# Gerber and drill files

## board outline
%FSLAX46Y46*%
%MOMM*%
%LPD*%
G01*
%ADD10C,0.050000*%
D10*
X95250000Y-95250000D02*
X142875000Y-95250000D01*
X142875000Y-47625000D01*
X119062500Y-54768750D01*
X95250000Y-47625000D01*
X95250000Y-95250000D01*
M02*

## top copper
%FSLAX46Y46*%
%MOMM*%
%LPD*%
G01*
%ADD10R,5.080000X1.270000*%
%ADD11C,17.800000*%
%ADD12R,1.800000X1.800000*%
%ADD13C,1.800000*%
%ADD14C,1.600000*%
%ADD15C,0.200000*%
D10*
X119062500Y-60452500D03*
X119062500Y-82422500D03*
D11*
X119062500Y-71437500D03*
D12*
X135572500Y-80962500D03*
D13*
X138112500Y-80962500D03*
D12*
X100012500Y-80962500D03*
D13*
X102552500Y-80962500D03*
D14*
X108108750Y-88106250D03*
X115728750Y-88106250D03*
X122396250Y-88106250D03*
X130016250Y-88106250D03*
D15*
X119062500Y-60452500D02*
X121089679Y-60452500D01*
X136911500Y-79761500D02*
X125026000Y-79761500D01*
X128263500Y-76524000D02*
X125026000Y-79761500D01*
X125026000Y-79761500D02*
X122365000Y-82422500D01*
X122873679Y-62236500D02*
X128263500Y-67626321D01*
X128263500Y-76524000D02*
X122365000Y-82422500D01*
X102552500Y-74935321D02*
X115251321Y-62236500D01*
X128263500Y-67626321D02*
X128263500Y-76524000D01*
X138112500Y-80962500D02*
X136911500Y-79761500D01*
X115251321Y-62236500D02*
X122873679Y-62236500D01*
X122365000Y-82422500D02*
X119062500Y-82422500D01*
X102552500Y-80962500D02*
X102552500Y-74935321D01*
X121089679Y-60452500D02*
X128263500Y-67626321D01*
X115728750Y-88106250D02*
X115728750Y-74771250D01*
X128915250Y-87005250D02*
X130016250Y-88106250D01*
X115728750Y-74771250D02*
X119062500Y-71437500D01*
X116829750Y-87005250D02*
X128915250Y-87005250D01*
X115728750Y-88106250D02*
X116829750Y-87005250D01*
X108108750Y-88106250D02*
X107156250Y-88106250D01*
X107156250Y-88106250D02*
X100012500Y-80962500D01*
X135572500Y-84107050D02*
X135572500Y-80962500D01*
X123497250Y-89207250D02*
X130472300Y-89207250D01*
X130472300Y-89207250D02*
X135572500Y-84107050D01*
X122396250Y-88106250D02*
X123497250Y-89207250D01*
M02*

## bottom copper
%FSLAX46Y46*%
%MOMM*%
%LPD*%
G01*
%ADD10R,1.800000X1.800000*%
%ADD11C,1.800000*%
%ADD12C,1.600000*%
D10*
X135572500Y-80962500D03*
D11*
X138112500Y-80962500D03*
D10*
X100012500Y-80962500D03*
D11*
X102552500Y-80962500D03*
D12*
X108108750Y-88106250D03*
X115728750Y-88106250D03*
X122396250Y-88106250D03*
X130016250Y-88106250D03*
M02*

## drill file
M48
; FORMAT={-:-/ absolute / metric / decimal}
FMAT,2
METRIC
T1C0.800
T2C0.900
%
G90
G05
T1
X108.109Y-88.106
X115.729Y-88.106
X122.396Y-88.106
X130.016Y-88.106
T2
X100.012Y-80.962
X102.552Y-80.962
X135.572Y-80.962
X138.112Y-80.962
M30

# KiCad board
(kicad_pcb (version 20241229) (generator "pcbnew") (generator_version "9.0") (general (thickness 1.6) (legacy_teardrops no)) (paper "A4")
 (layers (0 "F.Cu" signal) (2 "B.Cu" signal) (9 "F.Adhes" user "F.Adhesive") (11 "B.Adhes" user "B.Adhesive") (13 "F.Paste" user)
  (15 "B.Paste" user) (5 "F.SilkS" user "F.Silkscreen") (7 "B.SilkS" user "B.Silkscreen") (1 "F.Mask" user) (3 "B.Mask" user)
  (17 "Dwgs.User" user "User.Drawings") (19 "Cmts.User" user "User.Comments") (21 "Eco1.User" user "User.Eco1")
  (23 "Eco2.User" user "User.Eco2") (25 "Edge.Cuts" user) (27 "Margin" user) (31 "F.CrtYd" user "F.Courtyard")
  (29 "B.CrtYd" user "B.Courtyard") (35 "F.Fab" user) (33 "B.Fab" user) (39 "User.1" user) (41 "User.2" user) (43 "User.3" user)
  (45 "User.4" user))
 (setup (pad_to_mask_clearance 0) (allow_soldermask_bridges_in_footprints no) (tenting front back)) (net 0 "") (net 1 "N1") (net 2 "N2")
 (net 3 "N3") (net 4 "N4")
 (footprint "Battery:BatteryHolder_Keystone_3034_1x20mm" (layer "F.Cu") (at 119.0625 71.4375 -90)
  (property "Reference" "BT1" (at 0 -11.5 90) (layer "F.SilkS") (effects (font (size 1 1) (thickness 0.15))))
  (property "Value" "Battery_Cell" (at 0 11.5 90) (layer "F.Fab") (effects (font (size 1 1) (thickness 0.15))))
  (pad "1" smd rect (at -10.985 0 270) (size 1.27 5.08) (layers "F.Cu" "F.Mask" "F.Paste") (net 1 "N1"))
  (pad "1" smd rect (at 10.985 0 270) (size 1.27 5.08) (layers "F.Cu" "F.Mask" "F.Paste") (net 1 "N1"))
  (pad "2" smd circle (at 0 0 270) (size 17.8 17.8) (layers "F.Cu" "F.Mask") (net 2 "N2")))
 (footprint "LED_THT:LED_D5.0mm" (layer "F.Cu") (at 135.5725 80.9625)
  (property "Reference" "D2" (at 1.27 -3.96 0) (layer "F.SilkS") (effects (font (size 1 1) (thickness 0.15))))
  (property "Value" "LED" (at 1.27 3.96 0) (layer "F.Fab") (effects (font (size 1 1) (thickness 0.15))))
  (pad "1" thru_hole rect (at 0 0) (size 1.8 1.8) (drill 0.9) (layers "*.Cu" "*.Mask") (remove_unused_layers no) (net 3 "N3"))
  (pad "2" thru_hole circle (at 2.54 0) (size 1.8 1.8) (drill 0.9) (layers "*.Cu" "*.Mask") (remove_unused_layers no) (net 1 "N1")))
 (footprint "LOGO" (layer "F.Cu") (at 104.775 57.15)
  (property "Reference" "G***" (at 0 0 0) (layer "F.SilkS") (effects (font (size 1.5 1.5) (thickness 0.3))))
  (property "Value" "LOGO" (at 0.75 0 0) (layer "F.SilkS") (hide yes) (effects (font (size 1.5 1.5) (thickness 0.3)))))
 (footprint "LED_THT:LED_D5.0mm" (layer "F.Cu") (at 100.0125 80.9625)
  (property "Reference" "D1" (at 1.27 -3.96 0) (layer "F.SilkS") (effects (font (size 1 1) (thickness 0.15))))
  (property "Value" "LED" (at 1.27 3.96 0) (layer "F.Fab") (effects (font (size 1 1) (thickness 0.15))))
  (pad "1" thru_hole rect (at 0 0) (size 1.8 1.8) (drill 0.9) (layers "*.Cu" "*.Mask") (remove_unused_layers no) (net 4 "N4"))
  (pad "2" thru_hole circle (at 2.54 0) (size 1.8 1.8) (drill 0.9) (layers "*.Cu" "*.Mask") (remove_unused_layers no) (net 1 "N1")))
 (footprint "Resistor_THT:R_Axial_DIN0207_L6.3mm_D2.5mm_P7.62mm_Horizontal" (layer "F.Cu") (at 108.10875 88.10625)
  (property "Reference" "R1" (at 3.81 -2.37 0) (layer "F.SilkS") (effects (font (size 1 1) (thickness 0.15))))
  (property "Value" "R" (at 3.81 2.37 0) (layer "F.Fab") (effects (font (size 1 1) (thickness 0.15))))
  (pad "1" thru_hole circle (at 0 0) (size 1.6 1.6) (drill 0.8) (layers "*.Cu" "*.Mask") (remove_unused_layers no) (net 4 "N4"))
  (pad "2" thru_hole circle (at 7.62 0) (size 1.6 1.6) (drill 0.8) (layers "*.Cu" "*.Mask") (remove_unused_layers no) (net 2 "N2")))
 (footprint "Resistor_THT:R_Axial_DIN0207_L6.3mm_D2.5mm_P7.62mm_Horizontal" (layer "F.Cu") (at 122.39625 88.10625)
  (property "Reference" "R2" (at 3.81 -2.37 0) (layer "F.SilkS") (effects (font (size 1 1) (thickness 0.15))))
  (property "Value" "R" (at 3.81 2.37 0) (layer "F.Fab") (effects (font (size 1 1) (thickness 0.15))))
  (pad "1" thru_hole circle (at 0 0) (size 1.6 1.6) (drill 0.8) (layers "*.Cu" "*.Mask") (remove_unused_layers no) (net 3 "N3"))
  (pad "2" thru_hole circle (at 7.62 0) (size 1.6 1.6) (drill 0.8) (layers "*.Cu" "*.Mask") (remove_unused_layers no) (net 2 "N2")))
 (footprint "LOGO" (layer "F.Cu") (at 133.35 59.53125)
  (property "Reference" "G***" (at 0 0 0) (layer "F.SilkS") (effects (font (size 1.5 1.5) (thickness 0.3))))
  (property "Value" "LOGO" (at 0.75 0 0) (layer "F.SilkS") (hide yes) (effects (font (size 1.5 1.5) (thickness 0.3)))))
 (gr_poly
  (pts (xy 95.25 95.25) (xy 142.875 95.25) (xy 142.875 47.625) (xy 119.0625 54.76875) (xy 95.25 47.625)) (stroke (width 0.05) (type solid))
  (fill no) (layer "Edge.Cuts"))
 (segment (start 119.0625 60.4525) (end 121.089679 60.4525) (width 0.2) (layer "F.Cu") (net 1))
 (segment (start 136.9115 79.7615) (end 125.026 79.7615) (width 0.2) (layer "F.Cu") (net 1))
 (segment (start 128.2635 76.524) (end 125.026 79.7615) (width 0.2) (layer "F.Cu") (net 1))
 (segment (start 125.026 79.7615) (end 122.365 82.4225) (width 0.2) (layer "F.Cu") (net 1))
 (segment (start 122.873679 62.2365) (end 128.2635 67.626321) (width 0.2) (layer "F.Cu") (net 1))
 (segment (start 128.2635 76.524) (end 122.365 82.4225) (width 0.2) (layer "F.Cu") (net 1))
 (segment (start 102.5525 74.935321) (end 115.251321 62.2365) (width 0.2) (layer "F.Cu") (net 1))
 (segment (start 128.2635 67.626321) (end 128.2635 76.524) (width 0.2) (layer "F.Cu") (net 1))
 (segment (start 138.1125 80.9625) (end 136.9115 79.7615) (width 0.2) (layer "F.Cu") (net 1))
 (segment (start 115.251321 62.2365) (end 122.873679 62.2365) (width 0.2) (layer "F.Cu") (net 1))
 (segment (start 122.365 82.4225) (end 119.0625 82.4225) (width 0.2) (layer "F.Cu") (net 1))
 (segment (start 102.5525 80.9625) (end 102.5525 74.935321) (width 0.2) (layer "F.Cu") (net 1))
 (segment (start 121.089679 60.4525) (end 128.2635 67.626321) (width 0.2) (layer "F.Cu") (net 1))
 (segment (start 115.72875 88.10625) (end 115.72875 74.77125) (width 0.2) (layer "F.Cu") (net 2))
 (segment (start 128.91525 87.00525) (end 130.01625 88.10625) (width 0.2) (layer "F.Cu") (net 2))
 (segment (start 115.72875 74.77125) (end 119.0625 71.4375) (width 0.2) (layer "F.Cu") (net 2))
 (segment (start 116.82975 87.00525) (end 128.91525 87.00525) (width 0.2) (layer "F.Cu") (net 2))
 (segment (start 115.72875 88.10625) (end 116.82975 87.00525) (width 0.2) (layer "F.Cu") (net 2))
 (segment (start 108.10875 88.10625) (end 107.15625 88.10625) (width 0.2) (layer "F.Cu") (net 4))
 (segment (start 107.15625 88.10625) (end 100.0125 80.9625) (width 0.2) (layer "F.Cu") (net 4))
 (segment (start 135.5725 84.10705) (end 135.5725 80.9625) (width 0.2) (layer "F.Cu") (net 3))
 (segment (start 123.49725 89.20725) (end 130.4723 89.20725) (width 0.2) (layer "F.Cu") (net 3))
 (segment (start 130.4723 89.20725) (end 135.5725 84.10705) (width 0.2) (layer "F.Cu") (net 3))
 (segment (start 122.39625 88.10625) (end 123.49725 89.20725) (width 0.2) (layer "F.Cu") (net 3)))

